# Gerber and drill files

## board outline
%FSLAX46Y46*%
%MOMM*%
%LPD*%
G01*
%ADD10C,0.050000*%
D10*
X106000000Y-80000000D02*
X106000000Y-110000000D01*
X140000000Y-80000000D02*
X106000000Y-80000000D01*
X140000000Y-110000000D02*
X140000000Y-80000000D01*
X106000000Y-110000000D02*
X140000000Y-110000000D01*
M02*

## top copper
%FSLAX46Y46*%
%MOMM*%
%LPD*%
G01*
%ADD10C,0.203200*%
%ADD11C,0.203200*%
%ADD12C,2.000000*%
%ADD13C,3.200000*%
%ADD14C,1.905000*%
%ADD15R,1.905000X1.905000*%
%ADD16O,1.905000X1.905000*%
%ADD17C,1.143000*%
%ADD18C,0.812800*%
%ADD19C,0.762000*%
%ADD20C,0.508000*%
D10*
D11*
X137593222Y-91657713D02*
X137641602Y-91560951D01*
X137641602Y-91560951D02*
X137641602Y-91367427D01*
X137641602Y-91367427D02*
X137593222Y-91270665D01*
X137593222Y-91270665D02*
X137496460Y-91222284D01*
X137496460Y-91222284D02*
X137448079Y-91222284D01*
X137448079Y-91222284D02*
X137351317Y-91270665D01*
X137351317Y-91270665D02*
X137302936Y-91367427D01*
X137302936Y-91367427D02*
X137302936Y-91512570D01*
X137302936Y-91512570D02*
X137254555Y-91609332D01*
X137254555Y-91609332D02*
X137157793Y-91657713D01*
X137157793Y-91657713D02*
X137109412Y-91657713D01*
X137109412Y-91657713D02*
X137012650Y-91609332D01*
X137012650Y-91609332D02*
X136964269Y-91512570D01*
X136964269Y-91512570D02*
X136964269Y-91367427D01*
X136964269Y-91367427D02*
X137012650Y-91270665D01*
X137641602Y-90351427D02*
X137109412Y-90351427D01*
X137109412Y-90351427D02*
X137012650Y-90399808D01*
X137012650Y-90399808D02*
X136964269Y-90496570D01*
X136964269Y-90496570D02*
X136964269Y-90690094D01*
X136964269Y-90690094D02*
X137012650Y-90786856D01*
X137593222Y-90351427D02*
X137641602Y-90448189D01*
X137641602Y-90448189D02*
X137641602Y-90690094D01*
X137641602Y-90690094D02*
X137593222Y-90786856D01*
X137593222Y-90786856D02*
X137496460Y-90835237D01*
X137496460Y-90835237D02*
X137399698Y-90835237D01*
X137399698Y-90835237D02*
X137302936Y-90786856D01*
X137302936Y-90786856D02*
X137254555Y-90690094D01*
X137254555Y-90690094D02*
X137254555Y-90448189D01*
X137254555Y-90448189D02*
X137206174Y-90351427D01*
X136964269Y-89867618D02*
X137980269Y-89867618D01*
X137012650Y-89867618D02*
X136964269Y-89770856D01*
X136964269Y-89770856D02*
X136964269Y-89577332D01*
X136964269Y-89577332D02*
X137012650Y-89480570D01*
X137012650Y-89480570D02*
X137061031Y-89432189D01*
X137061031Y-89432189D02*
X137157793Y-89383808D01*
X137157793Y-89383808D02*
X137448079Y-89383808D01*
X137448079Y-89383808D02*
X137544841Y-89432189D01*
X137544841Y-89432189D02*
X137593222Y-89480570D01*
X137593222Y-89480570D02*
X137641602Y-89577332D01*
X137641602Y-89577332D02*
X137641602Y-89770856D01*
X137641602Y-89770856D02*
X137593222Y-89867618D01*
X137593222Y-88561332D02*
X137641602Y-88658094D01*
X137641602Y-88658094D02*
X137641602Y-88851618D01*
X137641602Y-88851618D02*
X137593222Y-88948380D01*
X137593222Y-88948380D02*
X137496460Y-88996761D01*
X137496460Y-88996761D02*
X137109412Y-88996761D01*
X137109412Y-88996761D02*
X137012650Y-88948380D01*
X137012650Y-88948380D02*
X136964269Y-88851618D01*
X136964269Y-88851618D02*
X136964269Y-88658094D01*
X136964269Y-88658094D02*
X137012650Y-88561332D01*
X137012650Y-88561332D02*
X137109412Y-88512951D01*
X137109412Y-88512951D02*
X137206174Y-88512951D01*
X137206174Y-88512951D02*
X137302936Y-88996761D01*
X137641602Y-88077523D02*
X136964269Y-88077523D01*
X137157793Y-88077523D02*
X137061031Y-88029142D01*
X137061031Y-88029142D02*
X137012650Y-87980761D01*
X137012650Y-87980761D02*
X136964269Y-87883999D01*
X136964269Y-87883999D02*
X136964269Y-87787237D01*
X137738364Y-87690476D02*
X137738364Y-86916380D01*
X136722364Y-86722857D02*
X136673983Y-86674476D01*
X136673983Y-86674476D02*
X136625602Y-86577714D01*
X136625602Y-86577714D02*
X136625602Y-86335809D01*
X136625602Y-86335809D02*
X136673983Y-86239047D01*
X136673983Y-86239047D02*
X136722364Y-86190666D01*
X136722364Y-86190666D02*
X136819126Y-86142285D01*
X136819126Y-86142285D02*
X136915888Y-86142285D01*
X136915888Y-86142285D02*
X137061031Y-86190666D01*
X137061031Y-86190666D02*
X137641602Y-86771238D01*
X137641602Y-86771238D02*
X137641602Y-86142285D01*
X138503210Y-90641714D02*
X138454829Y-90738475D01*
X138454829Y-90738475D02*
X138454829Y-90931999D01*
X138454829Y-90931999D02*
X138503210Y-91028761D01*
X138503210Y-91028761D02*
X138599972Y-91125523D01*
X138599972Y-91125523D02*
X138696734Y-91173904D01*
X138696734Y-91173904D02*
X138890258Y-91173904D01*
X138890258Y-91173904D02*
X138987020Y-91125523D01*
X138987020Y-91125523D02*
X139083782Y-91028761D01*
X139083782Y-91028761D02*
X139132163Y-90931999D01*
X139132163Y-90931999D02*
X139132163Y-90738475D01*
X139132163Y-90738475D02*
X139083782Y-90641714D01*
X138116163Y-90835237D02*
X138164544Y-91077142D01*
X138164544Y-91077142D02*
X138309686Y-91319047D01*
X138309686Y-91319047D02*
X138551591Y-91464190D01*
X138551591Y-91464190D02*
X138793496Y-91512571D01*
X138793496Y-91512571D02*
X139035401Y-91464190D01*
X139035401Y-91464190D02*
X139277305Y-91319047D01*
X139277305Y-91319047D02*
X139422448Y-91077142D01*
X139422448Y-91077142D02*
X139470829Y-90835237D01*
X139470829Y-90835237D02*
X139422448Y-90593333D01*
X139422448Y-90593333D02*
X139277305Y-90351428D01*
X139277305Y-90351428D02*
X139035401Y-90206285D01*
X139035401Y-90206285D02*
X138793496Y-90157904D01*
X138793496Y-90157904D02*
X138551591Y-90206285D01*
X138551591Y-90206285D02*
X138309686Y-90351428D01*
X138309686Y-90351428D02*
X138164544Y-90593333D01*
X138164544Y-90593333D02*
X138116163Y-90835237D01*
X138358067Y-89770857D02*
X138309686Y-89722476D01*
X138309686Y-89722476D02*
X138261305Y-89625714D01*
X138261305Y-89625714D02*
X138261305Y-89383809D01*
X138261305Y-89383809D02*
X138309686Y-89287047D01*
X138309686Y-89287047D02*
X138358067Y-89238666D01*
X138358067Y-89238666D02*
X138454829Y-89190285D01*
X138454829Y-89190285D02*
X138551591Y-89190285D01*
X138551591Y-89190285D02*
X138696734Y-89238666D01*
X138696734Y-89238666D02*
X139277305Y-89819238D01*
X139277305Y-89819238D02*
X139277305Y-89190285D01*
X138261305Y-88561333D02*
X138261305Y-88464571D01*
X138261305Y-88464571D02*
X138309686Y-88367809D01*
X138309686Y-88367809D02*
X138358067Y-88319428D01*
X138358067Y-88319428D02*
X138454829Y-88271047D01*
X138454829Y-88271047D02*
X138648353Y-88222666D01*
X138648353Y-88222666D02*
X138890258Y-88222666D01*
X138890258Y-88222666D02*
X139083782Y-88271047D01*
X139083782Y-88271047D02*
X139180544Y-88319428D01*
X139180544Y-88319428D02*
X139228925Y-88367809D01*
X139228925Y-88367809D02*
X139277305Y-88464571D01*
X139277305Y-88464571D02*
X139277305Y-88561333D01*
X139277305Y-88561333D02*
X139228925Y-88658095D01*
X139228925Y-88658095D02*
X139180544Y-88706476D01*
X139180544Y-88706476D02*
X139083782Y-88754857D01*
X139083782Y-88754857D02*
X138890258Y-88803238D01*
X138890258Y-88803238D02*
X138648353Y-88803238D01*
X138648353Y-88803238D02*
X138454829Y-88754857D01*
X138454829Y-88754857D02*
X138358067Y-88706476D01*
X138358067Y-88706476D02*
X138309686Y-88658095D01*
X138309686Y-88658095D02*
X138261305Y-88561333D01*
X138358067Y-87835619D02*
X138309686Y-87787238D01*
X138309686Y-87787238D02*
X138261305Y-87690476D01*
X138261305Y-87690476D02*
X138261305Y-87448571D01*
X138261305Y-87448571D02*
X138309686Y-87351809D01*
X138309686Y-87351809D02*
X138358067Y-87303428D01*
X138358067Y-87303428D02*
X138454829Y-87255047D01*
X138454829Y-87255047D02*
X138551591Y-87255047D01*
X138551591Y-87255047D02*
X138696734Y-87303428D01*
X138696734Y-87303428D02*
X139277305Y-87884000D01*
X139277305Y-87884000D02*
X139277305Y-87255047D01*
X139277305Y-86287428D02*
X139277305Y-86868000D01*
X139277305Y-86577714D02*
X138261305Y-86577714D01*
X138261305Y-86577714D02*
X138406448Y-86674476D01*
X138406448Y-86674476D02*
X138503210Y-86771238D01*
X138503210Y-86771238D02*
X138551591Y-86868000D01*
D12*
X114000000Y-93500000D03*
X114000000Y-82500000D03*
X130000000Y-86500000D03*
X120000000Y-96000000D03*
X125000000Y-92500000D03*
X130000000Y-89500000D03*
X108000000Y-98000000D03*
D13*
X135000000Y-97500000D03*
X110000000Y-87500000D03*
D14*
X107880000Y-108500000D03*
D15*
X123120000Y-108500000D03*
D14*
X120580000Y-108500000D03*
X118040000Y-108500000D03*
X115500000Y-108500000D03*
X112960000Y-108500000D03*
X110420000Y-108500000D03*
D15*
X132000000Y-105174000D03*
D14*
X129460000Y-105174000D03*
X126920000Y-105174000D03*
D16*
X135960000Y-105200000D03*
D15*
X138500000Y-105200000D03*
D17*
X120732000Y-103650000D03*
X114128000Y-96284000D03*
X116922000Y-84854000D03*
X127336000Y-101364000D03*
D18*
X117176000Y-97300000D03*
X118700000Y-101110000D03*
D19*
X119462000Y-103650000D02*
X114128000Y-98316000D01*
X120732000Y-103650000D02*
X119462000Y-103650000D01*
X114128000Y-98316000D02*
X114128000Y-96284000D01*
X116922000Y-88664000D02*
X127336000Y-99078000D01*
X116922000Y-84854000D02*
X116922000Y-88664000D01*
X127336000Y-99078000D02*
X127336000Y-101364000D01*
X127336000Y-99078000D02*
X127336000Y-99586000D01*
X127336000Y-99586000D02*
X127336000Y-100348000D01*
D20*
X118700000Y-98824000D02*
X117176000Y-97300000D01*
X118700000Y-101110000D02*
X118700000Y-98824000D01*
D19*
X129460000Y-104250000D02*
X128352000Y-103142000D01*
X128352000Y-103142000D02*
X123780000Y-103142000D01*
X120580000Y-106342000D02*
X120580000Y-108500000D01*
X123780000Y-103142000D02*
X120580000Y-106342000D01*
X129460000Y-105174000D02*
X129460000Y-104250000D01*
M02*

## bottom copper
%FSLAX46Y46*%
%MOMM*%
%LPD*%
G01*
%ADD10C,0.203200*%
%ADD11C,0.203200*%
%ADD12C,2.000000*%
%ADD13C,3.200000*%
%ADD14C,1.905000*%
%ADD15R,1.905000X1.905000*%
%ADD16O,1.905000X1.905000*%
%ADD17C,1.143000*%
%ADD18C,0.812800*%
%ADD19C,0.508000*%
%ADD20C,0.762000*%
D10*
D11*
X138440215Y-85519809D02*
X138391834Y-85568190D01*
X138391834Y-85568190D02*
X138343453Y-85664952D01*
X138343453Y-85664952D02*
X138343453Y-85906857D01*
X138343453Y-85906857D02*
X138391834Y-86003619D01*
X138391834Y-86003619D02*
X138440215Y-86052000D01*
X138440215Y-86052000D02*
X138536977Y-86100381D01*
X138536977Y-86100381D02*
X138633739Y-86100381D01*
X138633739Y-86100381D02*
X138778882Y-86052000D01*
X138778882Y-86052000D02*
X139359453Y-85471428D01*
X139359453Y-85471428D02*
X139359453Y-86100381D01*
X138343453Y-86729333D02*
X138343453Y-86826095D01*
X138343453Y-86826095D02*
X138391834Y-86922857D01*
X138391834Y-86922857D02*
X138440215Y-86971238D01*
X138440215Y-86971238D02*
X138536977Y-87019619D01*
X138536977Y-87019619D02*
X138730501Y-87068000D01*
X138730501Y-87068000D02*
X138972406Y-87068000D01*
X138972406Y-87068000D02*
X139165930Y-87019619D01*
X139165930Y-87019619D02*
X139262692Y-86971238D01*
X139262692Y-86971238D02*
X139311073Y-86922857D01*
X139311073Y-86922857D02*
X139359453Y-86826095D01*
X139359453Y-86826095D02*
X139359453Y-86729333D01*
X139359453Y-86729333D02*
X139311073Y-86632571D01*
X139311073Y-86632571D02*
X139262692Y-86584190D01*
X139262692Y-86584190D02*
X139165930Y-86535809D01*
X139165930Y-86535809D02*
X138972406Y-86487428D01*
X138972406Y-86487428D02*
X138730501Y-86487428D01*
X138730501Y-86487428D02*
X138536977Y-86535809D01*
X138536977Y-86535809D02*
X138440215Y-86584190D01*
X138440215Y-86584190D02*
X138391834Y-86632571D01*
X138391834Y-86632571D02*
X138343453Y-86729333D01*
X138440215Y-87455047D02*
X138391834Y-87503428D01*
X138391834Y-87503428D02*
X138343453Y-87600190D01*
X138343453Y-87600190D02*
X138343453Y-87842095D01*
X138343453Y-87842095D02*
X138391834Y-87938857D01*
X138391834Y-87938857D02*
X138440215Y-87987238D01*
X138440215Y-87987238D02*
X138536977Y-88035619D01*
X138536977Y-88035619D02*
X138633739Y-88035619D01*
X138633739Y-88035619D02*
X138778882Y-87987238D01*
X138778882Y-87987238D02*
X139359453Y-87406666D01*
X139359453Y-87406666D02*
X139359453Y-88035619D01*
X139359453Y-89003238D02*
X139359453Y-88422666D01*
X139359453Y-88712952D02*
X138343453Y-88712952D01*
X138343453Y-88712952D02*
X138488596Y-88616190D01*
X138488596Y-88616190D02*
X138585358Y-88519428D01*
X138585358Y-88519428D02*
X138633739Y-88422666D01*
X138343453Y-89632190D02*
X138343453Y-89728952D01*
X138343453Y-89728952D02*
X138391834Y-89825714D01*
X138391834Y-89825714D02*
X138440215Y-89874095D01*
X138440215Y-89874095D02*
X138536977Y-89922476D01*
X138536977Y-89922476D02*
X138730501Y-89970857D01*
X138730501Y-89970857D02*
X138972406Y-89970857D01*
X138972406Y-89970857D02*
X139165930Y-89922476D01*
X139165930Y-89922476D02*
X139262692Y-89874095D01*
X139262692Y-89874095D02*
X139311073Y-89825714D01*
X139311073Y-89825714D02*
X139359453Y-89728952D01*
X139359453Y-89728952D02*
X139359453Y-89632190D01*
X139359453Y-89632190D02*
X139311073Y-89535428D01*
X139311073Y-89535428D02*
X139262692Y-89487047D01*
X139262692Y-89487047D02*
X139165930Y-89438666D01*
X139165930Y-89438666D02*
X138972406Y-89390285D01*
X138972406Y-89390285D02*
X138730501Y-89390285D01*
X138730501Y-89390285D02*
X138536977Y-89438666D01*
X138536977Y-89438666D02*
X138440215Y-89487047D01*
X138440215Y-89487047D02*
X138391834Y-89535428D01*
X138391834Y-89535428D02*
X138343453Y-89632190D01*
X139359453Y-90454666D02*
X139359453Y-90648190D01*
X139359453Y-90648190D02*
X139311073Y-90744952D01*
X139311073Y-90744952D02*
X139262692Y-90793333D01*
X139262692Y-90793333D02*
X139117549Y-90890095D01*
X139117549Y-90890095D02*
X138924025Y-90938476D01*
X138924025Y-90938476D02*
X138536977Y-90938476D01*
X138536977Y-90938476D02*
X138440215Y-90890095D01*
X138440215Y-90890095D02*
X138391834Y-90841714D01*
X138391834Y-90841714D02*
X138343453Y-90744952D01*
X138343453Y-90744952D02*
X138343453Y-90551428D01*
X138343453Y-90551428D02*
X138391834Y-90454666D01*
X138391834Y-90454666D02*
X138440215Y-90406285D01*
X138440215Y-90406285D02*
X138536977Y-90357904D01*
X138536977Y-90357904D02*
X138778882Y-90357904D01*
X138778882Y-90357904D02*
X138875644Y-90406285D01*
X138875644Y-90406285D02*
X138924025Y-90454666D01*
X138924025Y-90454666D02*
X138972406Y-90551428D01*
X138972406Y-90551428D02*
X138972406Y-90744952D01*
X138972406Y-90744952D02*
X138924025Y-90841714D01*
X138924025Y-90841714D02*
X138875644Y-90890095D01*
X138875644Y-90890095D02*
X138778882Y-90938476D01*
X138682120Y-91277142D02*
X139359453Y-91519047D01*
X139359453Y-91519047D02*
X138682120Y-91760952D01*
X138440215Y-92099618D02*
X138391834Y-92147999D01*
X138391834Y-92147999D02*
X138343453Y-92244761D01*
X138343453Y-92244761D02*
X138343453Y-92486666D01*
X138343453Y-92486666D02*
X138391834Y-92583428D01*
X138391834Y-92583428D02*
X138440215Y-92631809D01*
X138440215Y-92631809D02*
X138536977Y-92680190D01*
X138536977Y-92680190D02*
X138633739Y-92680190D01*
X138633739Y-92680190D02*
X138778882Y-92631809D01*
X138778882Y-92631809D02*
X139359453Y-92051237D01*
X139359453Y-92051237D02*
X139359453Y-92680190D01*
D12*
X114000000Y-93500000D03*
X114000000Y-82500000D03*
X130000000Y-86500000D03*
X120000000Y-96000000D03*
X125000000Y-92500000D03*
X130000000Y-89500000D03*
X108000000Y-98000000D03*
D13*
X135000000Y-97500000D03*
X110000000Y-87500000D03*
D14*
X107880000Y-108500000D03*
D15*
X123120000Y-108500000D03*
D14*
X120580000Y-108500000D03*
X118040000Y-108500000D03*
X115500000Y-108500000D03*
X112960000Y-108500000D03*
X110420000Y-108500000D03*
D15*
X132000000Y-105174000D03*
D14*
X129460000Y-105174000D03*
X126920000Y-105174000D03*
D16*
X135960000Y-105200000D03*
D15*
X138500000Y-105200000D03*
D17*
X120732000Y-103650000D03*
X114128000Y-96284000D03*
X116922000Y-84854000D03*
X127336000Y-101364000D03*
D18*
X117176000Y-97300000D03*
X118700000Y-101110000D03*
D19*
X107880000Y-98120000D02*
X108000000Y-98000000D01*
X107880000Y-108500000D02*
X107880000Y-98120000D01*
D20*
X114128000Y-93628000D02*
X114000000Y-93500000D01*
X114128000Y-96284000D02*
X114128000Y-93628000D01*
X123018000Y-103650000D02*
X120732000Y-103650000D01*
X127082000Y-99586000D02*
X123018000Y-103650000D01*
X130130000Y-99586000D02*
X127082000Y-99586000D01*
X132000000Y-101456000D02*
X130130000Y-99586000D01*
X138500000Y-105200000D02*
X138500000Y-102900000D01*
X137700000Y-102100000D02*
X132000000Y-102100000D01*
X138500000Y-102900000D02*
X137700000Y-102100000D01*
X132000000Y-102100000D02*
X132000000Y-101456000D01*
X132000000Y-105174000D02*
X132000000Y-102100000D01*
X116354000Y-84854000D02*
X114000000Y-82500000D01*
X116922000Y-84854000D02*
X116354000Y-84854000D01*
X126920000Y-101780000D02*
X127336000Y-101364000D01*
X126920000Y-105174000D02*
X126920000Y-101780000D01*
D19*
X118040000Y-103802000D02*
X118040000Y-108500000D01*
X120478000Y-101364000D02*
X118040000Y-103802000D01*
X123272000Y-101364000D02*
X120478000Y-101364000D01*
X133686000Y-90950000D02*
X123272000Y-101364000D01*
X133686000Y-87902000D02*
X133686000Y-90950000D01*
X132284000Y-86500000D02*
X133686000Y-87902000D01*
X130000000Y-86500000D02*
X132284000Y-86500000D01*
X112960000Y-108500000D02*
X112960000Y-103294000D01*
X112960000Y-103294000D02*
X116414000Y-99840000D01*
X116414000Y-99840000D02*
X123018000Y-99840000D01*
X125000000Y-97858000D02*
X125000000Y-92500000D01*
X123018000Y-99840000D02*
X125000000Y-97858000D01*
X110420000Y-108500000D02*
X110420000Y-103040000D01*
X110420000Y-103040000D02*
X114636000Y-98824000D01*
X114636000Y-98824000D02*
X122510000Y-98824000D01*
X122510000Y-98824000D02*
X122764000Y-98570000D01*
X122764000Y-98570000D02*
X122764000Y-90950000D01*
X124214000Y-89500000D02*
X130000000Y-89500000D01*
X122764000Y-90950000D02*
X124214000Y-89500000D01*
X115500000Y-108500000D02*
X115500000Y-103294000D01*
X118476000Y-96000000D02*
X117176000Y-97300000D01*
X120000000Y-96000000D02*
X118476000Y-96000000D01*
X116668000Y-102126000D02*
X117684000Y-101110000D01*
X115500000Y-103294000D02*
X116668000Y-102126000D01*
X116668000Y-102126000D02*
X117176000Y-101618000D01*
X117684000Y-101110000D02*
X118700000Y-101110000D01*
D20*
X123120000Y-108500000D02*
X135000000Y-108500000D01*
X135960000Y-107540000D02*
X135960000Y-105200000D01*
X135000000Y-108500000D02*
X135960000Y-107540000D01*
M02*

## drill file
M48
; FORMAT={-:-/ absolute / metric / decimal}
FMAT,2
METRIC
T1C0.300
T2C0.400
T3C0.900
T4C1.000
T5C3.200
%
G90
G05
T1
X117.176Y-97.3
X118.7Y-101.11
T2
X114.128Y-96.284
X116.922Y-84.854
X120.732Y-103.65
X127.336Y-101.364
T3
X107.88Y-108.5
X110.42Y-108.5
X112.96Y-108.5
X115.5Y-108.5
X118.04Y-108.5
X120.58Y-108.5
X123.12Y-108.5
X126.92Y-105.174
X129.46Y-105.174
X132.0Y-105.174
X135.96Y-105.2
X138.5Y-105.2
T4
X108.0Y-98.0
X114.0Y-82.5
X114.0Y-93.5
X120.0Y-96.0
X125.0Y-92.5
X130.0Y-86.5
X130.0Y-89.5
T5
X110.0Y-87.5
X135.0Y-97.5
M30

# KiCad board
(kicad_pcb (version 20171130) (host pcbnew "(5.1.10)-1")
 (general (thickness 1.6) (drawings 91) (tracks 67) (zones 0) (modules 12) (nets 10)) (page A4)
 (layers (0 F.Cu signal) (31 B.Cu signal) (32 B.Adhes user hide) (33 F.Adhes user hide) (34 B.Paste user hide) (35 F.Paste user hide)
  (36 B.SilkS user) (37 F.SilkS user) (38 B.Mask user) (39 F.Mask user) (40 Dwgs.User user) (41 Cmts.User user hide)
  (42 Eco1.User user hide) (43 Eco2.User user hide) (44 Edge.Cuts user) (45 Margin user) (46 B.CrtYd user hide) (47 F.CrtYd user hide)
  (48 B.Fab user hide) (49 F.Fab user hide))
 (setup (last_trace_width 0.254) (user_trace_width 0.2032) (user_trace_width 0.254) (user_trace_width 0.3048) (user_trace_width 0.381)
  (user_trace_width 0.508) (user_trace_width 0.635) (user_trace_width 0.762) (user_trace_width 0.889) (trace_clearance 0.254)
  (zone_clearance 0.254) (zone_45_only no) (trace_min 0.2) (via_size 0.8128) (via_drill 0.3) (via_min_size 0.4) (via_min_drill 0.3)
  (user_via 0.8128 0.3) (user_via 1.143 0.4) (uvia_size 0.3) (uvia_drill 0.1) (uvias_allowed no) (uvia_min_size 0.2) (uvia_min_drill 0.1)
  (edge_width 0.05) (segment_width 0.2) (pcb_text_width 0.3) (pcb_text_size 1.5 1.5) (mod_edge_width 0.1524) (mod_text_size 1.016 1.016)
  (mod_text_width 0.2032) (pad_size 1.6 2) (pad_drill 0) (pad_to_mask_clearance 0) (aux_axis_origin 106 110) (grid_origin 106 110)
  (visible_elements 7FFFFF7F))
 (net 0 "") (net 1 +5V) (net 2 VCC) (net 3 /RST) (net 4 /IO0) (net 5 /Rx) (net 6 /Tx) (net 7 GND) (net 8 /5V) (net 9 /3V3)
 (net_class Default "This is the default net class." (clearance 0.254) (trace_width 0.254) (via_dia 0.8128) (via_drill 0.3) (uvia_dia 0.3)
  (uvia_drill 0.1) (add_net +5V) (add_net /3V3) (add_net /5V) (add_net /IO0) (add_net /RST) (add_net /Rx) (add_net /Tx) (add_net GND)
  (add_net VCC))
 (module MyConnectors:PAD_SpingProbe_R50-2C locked (layer F.Cu) (at 114 93.5)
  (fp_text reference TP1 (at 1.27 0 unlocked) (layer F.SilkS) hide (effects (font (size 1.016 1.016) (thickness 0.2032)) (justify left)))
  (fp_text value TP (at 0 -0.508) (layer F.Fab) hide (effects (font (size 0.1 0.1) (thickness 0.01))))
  (pad 1 thru_hole circle (at 0 0) (size 2 2) (drill 1) (layers *.Cu *.Mask) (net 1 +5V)))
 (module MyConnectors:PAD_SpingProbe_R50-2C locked (layer F.Cu) (at 114 82.5)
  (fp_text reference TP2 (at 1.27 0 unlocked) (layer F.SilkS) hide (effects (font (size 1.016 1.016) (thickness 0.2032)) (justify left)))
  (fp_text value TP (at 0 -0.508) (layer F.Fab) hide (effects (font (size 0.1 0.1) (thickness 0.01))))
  (pad 1 thru_hole circle (at 0 0) (size 2 2) (drill 1) (layers *.Cu *.Mask) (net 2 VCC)))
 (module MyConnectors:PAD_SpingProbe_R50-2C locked (layer F.Cu) (at 130 86.5)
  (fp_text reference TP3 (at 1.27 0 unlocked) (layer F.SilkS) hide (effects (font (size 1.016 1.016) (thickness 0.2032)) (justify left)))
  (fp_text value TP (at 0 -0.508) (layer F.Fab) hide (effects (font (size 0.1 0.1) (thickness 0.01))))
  (pad 1 thru_hole circle (at 0 0) (size 2 2) (drill 1) (layers *.Cu *.Mask) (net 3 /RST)))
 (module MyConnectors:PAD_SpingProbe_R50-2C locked (layer F.Cu) (at 120 96)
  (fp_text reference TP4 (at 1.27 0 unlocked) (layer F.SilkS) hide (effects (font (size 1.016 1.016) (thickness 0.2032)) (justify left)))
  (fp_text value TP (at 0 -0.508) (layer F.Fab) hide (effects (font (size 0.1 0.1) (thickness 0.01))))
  (pad 1 thru_hole circle (at 0 0) (size 2 2) (drill 1) (layers *.Cu *.Mask) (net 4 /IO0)))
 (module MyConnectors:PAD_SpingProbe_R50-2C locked (layer F.Cu) (at 125 92.5)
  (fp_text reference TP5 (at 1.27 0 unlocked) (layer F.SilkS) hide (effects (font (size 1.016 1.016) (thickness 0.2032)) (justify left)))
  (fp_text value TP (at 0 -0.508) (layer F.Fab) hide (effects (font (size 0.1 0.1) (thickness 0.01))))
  (pad 1 thru_hole circle (at 0 0) (size 2 2) (drill 1) (layers *.Cu *.Mask) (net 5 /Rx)))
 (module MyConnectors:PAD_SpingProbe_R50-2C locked (layer F.Cu) (at 130 89.5)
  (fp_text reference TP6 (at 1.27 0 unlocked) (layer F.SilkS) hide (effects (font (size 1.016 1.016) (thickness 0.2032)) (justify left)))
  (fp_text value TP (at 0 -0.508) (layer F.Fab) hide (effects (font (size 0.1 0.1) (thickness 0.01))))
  (pad 1 thru_hole circle (at 0 0) (size 2 2) (drill 1) (layers *.Cu *.Mask) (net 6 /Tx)))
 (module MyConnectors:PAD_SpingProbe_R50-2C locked (layer F.Cu) (at 108 98)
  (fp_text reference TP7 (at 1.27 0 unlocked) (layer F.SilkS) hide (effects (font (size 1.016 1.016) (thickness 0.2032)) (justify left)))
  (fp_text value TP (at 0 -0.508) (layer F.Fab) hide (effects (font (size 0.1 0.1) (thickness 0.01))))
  (pad 1 thru_hole circle (at 0 0) (size 2 2) (drill 1) (layers *.Cu *.Mask) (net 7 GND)))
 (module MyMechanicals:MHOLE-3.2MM (layer F.Cu) (at 135 97.5)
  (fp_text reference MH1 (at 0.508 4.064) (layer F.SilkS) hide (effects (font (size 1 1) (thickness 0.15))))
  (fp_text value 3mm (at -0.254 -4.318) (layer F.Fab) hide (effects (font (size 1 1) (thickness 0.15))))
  (pad x thru_hole circle (at 0 0) (size 3.2 3.2) (drill 3.2) (layers *.Cu *.Mask F.SilkS)))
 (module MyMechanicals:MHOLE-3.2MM (layer F.Cu) (at 110 87.5)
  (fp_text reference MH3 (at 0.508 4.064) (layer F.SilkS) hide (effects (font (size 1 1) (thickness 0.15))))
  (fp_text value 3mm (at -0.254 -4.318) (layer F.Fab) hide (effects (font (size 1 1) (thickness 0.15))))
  (pad x thru_hole circle (at 0 0) (size 3.2 3.2) (drill 3.2) (layers *.Cu *.Mask F.SilkS)))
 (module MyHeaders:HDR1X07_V (layer F.Cu) (at 123.12 108.5 270)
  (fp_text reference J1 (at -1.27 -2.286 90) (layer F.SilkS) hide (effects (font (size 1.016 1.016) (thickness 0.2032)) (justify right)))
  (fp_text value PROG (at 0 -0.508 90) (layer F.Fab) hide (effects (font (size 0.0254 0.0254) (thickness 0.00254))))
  (pad 7 thru_hole circle (at 0 15.24 270) (size 1.905 1.905) (drill 0.9) (layers *.Cu *.Mask) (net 7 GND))
  (pad 1 thru_hole rect (at 0 0 270) (size 1.905 1.905) (drill 0.9) (layers *.Cu *.Mask) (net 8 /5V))
  (pad 2 thru_hole circle (at 0 2.54 270) (size 1.905 1.905) (drill 0.9) (layers *.Cu *.Mask) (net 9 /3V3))
  (pad 3 thru_hole circle (at 0 5.08 270) (size 1.905 1.905) (drill 0.9) (layers *.Cu *.Mask) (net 3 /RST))
  (pad 4 thru_hole circle (at 0 7.62 270) (size 1.905 1.905) (drill 0.9) (layers *.Cu *.Mask) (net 4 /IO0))
  (pad 5 thru_hole circle (at 0 10.16 270) (size 1.905 1.905) (drill 0.9) (layers *.Cu *.Mask) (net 5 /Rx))
  (pad 6 thru_hole circle (at 0 12.7 270) (size 1.905 1.905) (drill 0.9) (layers *.Cu *.Mask) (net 6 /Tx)))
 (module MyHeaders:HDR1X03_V (layer F.Cu) (at 132 105.174 270)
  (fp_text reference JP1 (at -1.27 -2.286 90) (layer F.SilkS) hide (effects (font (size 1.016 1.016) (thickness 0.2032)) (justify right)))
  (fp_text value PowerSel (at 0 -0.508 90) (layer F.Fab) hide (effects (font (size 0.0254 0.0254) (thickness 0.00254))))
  (pad 1 thru_hole rect (at 0 0 270) (size 1.905 1.905) (drill 0.9) (layers *.Cu *.Mask) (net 1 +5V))
  (pad 2 thru_hole circle (at 0 2.54 270) (size 1.905 1.905) (drill 0.9) (layers *.Cu *.Mask) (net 9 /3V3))
  (pad 3 thru_hole circle (at 0 5.08 270) (size 1.905 1.905) (drill 0.9) (layers *.Cu *.Mask) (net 2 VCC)))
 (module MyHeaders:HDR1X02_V (layer F.Cu) (at 138.5 105.2 270)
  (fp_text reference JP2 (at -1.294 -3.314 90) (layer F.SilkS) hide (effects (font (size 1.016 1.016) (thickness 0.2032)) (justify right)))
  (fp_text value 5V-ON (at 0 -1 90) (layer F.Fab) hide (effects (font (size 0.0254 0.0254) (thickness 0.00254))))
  (pad 2 thru_hole oval (at 0 2.54 270) (size 1.905 1.905) (drill 0.9) (layers *.Cu *.Mask) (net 8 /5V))
  (pad 1 thru_hole rect (at 0 0 270) (size 1.905 1.905) (drill 0.9) (layers *.Cu *.Mask) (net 1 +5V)))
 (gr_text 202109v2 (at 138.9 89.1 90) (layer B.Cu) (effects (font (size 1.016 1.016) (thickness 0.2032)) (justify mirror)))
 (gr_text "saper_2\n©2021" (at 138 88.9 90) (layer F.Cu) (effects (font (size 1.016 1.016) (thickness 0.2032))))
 (gr_line (start 106 80) (end 106 110) (layer Edge.Cuts) (width 0.05))
 (gr_line (start 140 80) (end 106 80) (layer Edge.Cuts) (width 0.05))
 (gr_line (start 140 110) (end 140 80) (layer Edge.Cuts) (width 0.05))
 (gr_line (start 106 110) (end 140 110) (layer Edge.Cuts) (width 0.05))
 (segment (start 107.88 98.12) (end 108 98) (width 0.508) (layer B.Cu) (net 7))
 (segment (start 107.88 108.5) (end 107.88 98.12) (width 0.508) (layer B.Cu) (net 7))
 (via (at 120.732 103.65) (size 1.143) (drill 0.4) (layers F.Cu B.Cu) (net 1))
 (segment (start 119.462 103.65) (end 114.128 98.316) (width 0.762) (layer F.Cu) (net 1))
 (segment (start 120.732 103.65) (end 119.462 103.65) (width 0.762) (layer F.Cu) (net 1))
 (segment (start 114.128 98.316) (end 114.128 96.284) (width 0.762) (layer F.Cu) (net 1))
 (via (at 114.128 96.284) (size 1.143) (drill 0.4) (layers F.Cu B.Cu) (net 1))
 (segment (start 114.128 93.628) (end 114 93.5) (width 0.762) (layer B.Cu) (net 1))
 (segment (start 114.128 96.284) (end 114.128 93.628) (width 0.762) (layer B.Cu) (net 1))
 (segment (start 123.018 103.65) (end 120.732 103.65) (width 0.762) (layer B.Cu) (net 1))
 (segment (start 127.082 99.586) (end 123.018 103.65) (width 0.762) (layer B.Cu) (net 1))
 (segment (start 130.13 99.586) (end 127.082 99.586) (width 0.762) (layer B.Cu) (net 1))
 (segment (start 132 101.456) (end 130.13 99.586) (width 0.762) (layer B.Cu) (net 1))
 (segment (start 138.5 105.2) (end 138.5 102.9) (width 0.762) (layer B.Cu) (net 1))
 (segment (start 137.7 102.1) (end 132 102.1) (width 0.762) (layer B.Cu) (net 1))
 (segment (start 138.5 102.9) (end 137.7 102.1) (width 0.762) (layer B.Cu) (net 1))
 (segment (start 132 102.1) (end 132 101.456) (width 0.762) (layer B.Cu) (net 1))
 (segment (start 132 105.174) (end 132 102.1) (width 0.762) (layer B.Cu) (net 1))
 (via (at 116.922 84.854) (size 1.143) (drill 0.4) (layers F.Cu B.Cu) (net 2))
 (segment (start 116.354 84.854) (end 114 82.5) (width 0.762) (layer B.Cu) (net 2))
 (segment (start 116.922 84.854) (end 116.354 84.854) (width 0.762) (layer B.Cu) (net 2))
 (segment (start 116.922 88.664) (end 127.336 99.078) (width 0.762) (layer F.Cu) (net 2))
 (segment (start 116.922 84.854) (end 116.922 88.664) (width 0.762) (layer F.Cu) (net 2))
 (segment (start 127.336 99.078) (end 127.336 101.364) (width 0.762) (layer F.Cu) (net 2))
 (via (at 127.336 101.364) (size 1.143) (drill 0.4) (layers F.Cu B.Cu) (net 2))
 (segment (start 127.336 99.078) (end 127.336 99.586) (width 0.762) (layer F.Cu) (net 2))
 (segment (start 127.336 99.586) (end 127.336 100.348) (width 0.762) (layer F.Cu) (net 2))
 (segment (start 126.92 101.78) (end 127.336 101.364) (width 0.762) (layer B.Cu) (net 2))
 (segment (start 126.92 105.174) (end 126.92 101.78) (width 0.762) (layer B.Cu) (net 2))
 (segment (start 118.04 103.802) (end 118.04 108.5) (width 0.508) (layer B.Cu) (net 3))
 (segment (start 120.478 101.364) (end 118.04 103.802) (width 0.508) (layer B.Cu) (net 3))
 (segment (start 123.272 101.364) (end 120.478 101.364) (width 0.508) (layer B.Cu) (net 3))
 (segment (start 133.686 90.95) (end 123.272 101.364) (width 0.508) (layer B.Cu) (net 3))
 (segment (start 133.686 87.902) (end 133.686 90.95) (width 0.508) (layer B.Cu) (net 3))
 (segment (start 132.284 86.5) (end 133.686 87.902) (width 0.508) (layer B.Cu) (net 3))
 (segment (start 130 86.5) (end 132.284 86.5) (width 0.508) (layer B.Cu) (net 3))
 (segment (start 112.96 108.5) (end 112.96 103.294) (width 0.508) (layer B.Cu) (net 5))
 (segment (start 112.96 103.294) (end 116.414 99.84) (width 0.508) (layer B.Cu) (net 5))
 (segment (start 116.414 99.84) (end 123.018 99.84) (width 0.508) (layer B.Cu) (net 5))
 (segment (start 125 97.858) (end 125 92.5) (width 0.508) (layer B.Cu) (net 5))
 (segment (start 123.018 99.84) (end 125 97.858) (width 0.508) (layer B.Cu) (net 5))
 (segment (start 110.42 108.5) (end 110.42 103.04) (width 0.508) (layer B.Cu) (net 6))
 (segment (start 110.42 103.04) (end 114.636 98.824) (width 0.508) (layer B.Cu) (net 6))
 (segment (start 114.636 98.824) (end 122.51 98.824) (width 0.508) (layer B.Cu) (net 6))
 (segment (start 122.51 98.824) (end 122.764 98.57) (width 0.508) (layer B.Cu) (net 6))
 (segment (start 122.764 98.57) (end 122.764 90.95) (width 0.508) (layer B.Cu) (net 6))
 (segment (start 124.214 89.5) (end 130 89.5) (width 0.508) (layer B.Cu) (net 6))
 (segment (start 122.764 90.95) (end 124.214 89.5) (width 0.508) (layer B.Cu) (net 6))
 (segment (start 115.5 108.5) (end 115.5 103.294) (width 0.508) (layer B.Cu) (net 4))
 (via (at 117.176 97.3) (size 0.8128) (drill 0.3) (layers F.Cu B.Cu) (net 4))
 (segment (start 118.476 96) (end 117.176 97.3) (width 0.508) (layer B.Cu) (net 4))
 (segment (start 120 96) (end 118.476 96) (width 0.508) (layer B.Cu) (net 4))
 (segment (start 116.668 102.126) (end 117.684 101.11) (width 0.508) (layer B.Cu) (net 4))
 (segment (start 115.5 103.294) (end 116.668 102.126) (width 0.508) (layer B.Cu) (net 4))
 (segment (start 116.668 102.126) (end 117.176 101.618) (width 0.508) (layer B.Cu) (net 4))
 (via (at 118.7 101.11) (size 0.8128) (drill 0.3) (layers F.Cu B.Cu) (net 4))
 (segment (start 117.684 101.11) (end 118.7 101.11) (width 0.508) (layer B.Cu) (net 4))
 (segment (start 118.7 98.824) (end 117.176 97.3) (width 0.508) (layer F.Cu) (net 4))
 (segment (start 118.7 101.11) (end 118.7 98.824) (width 0.508) (layer F.Cu) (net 4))
 (segment (start 123.12 108.5) (end 135 108.5) (width 0.762) (layer B.Cu) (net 8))
 (segment (start 135.96 107.54) (end 135.96 105.2) (width 0.762) (layer B.Cu) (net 8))
 (segment (start 135 108.5) (end 135.96 107.54) (width 0.762) (layer B.Cu) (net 8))
 (segment (start 129.46 104.25) (end 128.352 103.142) (width 0.762) (layer F.Cu) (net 9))
 (segment (start 128.352 103.142) (end 123.78 103.142) (width 0.762) (layer F.Cu) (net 9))
 (segment (start 120.58 106.342) (end 120.58 108.5) (width 0.762) (layer F.Cu) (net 9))
 (segment (start 123.78 103.142) (end 120.58 106.342) (width 0.762) (layer F.Cu) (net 9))
 (segment (start 129.46 105.174) (end 129.46 104.25) (width 0.762) (layer F.Cu) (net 9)))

